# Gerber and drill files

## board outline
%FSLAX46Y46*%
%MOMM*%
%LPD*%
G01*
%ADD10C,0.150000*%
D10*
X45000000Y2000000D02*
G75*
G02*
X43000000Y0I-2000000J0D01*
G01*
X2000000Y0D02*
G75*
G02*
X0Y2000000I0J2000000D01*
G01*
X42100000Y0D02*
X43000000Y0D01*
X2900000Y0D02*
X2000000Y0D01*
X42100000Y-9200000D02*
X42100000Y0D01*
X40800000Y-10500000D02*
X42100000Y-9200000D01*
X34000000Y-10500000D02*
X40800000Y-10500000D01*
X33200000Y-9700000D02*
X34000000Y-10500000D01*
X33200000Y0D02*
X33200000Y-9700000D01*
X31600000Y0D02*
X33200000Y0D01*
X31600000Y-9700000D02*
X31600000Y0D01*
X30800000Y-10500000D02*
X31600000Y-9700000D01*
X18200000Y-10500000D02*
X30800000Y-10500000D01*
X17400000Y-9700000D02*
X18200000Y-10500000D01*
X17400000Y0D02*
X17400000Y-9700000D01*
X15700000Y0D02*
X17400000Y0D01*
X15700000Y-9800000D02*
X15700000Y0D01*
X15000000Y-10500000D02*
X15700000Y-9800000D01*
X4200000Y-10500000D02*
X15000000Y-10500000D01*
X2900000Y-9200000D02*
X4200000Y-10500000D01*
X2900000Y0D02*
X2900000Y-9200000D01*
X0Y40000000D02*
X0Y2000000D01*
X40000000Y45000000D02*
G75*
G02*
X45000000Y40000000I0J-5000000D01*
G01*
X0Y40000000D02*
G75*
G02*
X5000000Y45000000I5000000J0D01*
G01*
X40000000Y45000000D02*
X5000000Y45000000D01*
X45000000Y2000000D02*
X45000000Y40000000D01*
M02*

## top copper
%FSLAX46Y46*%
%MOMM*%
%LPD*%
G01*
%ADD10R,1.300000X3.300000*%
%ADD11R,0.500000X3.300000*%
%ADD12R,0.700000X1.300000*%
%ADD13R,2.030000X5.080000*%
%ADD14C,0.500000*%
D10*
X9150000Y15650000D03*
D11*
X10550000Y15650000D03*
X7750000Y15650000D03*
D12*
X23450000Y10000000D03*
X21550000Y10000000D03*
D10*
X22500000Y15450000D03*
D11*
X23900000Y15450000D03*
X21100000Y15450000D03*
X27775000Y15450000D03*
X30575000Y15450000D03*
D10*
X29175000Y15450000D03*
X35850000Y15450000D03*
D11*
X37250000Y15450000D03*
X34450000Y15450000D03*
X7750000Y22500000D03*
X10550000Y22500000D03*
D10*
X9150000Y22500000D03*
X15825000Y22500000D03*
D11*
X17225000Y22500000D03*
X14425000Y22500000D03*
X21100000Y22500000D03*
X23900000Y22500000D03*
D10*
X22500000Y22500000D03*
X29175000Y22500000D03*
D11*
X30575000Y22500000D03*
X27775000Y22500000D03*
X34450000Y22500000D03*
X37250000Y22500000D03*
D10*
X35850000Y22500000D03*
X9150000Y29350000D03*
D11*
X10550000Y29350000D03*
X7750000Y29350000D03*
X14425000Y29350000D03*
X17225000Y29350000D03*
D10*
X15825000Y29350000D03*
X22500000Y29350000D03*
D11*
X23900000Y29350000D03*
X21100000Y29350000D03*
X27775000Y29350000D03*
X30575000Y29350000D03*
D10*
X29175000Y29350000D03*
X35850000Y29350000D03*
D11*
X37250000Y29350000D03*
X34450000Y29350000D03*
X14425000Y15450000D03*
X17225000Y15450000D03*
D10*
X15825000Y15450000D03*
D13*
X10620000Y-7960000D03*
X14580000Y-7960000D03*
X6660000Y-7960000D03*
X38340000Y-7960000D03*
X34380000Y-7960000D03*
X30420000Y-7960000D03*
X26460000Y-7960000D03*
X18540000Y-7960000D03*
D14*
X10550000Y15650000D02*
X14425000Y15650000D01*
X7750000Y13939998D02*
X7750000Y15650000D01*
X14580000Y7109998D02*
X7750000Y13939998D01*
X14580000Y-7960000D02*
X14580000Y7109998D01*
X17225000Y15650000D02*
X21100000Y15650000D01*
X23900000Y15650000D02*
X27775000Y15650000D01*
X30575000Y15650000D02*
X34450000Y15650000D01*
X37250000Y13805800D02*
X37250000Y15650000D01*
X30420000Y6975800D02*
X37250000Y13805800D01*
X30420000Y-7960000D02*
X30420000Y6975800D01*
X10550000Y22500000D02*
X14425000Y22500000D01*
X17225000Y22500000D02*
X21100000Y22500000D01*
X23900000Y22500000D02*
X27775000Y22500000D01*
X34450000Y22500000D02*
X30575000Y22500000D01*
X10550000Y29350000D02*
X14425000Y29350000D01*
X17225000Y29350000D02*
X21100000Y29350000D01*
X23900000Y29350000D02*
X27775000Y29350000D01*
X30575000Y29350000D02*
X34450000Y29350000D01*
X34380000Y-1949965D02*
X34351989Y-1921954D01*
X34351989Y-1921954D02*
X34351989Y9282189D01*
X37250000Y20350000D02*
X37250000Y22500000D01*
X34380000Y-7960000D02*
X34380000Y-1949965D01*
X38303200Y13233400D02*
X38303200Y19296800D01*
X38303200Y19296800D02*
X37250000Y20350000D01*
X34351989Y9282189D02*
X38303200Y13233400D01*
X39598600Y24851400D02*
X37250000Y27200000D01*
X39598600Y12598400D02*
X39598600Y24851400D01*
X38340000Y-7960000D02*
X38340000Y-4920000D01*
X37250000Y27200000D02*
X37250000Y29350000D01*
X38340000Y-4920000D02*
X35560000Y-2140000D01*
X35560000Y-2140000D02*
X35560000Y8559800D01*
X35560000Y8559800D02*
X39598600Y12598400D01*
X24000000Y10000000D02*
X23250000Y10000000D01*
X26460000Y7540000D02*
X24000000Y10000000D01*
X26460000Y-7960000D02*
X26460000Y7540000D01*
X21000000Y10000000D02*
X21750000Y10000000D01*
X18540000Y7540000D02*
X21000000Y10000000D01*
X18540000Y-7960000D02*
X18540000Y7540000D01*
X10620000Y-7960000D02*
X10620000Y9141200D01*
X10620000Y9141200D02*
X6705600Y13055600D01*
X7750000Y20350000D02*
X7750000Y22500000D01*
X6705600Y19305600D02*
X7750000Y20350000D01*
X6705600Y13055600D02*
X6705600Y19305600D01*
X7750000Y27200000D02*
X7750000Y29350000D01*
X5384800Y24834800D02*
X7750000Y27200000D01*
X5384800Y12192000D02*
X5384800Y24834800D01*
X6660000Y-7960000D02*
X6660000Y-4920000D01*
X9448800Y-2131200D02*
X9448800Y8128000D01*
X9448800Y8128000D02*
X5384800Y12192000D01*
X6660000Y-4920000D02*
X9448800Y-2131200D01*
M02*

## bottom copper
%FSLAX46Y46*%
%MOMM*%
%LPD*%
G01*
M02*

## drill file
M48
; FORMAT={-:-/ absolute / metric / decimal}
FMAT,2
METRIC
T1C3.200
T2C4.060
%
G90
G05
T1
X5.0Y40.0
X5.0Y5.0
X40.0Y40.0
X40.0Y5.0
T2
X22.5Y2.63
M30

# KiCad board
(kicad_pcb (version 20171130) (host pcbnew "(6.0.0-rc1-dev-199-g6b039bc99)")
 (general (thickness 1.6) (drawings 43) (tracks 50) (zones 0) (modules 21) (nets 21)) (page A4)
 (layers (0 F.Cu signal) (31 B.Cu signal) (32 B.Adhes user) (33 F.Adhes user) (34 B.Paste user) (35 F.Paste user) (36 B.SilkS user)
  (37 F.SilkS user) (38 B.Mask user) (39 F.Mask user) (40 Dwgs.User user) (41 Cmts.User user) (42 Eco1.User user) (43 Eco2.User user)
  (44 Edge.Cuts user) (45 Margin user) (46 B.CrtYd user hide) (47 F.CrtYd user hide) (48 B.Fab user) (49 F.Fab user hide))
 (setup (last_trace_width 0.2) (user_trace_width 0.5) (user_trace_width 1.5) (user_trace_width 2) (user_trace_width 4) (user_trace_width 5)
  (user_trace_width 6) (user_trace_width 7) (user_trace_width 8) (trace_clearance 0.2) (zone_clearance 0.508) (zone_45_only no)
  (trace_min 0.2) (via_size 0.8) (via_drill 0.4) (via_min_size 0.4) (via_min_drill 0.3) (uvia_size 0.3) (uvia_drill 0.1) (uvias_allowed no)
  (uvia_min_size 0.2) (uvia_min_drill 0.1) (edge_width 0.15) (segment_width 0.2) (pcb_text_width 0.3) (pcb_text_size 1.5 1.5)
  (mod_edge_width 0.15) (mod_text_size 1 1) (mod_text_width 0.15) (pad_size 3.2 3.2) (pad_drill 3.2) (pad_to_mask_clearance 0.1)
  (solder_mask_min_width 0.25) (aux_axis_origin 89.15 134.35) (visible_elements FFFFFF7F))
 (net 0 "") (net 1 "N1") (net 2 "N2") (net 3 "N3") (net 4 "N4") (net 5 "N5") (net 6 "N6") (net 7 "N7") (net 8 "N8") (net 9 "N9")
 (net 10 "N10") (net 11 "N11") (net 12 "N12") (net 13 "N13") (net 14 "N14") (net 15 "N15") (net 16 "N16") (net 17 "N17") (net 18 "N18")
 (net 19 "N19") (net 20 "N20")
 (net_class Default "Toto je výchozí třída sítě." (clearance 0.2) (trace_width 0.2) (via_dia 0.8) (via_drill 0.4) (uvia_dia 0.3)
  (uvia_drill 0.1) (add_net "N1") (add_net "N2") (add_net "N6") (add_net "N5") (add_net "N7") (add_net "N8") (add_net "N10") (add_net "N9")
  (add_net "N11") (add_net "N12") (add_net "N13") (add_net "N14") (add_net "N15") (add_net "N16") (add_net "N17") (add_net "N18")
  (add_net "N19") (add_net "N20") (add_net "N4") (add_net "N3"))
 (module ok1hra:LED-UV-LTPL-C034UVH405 (layer F.Cu) (at 9.15 -15.65 180)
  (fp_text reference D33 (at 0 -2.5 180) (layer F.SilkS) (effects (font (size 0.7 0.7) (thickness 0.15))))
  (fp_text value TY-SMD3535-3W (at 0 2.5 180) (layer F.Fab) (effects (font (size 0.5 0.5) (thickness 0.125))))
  (pad 3 smd rect (at 0 0 180) (size 1.3 3.3) (layers F.Cu F.Paste F.Mask))
  (pad 1 smd rect (at -1.4 0 180) (size 0.5 3.3) (layers F.Cu F.Paste F.Mask) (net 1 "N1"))
  (pad 2 smd rect (at 1.4 0 180) (size 0.5 3.3) (layers F.Cu F.Paste F.Mask) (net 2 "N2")))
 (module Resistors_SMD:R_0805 (layer F.Cu) (at 22.5 -10 180)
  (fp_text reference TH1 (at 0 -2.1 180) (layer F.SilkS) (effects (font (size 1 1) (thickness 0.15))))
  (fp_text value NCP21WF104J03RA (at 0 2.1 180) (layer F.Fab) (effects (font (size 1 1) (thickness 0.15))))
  (pad 1 smd rect (at -0.95 0 180) (size 0.7 1.3) (layers F.Cu F.Paste F.Mask) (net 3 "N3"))
  (pad 2 smd rect (at 0.95 0 180) (size 0.7 1.3) (layers F.Cu F.Paste F.Mask) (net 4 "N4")))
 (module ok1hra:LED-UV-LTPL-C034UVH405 (layer F.Cu) (at 22.5 -15.45 180)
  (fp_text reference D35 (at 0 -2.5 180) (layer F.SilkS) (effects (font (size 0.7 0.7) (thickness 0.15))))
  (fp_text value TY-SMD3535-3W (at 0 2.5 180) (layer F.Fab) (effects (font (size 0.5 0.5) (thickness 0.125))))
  (pad 3 smd rect (at 0 0 180) (size 1.3 3.3) (layers F.Cu F.Paste F.Mask))
  (pad 1 smd rect (at -1.4 0 180) (size 0.5 3.3) (layers F.Cu F.Paste F.Mask) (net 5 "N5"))
  (pad 2 smd rect (at 1.4 0 180) (size 0.5 3.3) (layers F.Cu F.Paste F.Mask) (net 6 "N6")))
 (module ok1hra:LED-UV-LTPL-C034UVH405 (layer F.Cu) (at 29.175 -15.45 180)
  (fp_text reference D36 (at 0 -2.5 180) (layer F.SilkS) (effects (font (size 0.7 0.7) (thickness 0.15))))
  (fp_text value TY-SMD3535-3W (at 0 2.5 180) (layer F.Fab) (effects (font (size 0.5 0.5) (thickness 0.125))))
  (pad 2 smd rect (at 1.4 0 180) (size 0.5 3.3) (layers F.Cu F.Paste F.Mask) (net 5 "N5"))
  (pad 1 smd rect (at -1.4 0 180) (size 0.5 3.3) (layers F.Cu F.Paste F.Mask) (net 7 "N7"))
  (pad 3 smd rect (at 0 0 180) (size 1.3 3.3) (layers F.Cu F.Paste F.Mask)))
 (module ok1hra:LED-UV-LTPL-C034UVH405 (layer F.Cu) (at 35.85 -15.45 180)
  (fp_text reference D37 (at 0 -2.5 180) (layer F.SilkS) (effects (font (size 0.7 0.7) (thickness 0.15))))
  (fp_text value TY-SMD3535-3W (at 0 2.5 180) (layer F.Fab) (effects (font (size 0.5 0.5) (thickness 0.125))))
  (pad 3 smd rect (at 0 0 180) (size 1.3 3.3) (layers F.Cu F.Paste F.Mask))
  (pad 1 smd rect (at -1.4 0 180) (size 0.5 3.3) (layers F.Cu F.Paste F.Mask) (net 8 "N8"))
  (pad 2 smd rect (at 1.4 0 180) (size 0.5 3.3) (layers F.Cu F.Paste F.Mask) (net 7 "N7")))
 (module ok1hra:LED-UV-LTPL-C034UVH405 (layer F.Cu) (at 9.15 -22.5 180)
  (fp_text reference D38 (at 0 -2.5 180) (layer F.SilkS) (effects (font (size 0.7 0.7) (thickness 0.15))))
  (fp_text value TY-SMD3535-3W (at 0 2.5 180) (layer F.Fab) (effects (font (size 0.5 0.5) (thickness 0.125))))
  (pad 2 smd rect (at 1.4 0 180) (size 0.5 3.3) (layers F.Cu F.Paste F.Mask) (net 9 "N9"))
  (pad 1 smd rect (at -1.4 0 180) (size 0.5 3.3) (layers F.Cu F.Paste F.Mask) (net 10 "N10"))
  (pad 3 smd rect (at 0 0 180) (size 1.3 3.3) (layers F.Cu F.Paste F.Mask)))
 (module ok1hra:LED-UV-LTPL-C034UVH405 (layer F.Cu) (at 15.825 -22.5 180)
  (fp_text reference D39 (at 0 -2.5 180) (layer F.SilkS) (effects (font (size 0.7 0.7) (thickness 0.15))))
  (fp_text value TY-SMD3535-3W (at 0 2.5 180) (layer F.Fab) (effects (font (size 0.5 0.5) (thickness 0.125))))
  (pad 3 smd rect (at 0 0 180) (size 1.3 3.3) (layers F.Cu F.Paste F.Mask))
  (pad 1 smd rect (at -1.4 0 180) (size 0.5 3.3) (layers F.Cu F.Paste F.Mask) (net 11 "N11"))
  (pad 2 smd rect (at 1.4 0 180) (size 0.5 3.3) (layers F.Cu F.Paste F.Mask) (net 10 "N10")))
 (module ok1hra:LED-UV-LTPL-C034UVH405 (layer F.Cu) (at 22.5 -22.5 180)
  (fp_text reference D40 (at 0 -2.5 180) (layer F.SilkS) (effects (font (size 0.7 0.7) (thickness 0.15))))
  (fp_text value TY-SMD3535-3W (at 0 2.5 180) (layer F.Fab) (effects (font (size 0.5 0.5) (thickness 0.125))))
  (pad 2 smd rect (at 1.4 0 180) (size 0.5 3.3) (layers F.Cu F.Paste F.Mask) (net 11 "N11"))
  (pad 1 smd rect (at -1.4 0 180) (size 0.5 3.3) (layers F.Cu F.Paste F.Mask) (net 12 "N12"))
  (pad 3 smd rect (at 0 0 180) (size 1.3 3.3) (layers F.Cu F.Paste F.Mask)))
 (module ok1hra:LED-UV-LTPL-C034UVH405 (layer F.Cu) (at 29.175 -22.5 180)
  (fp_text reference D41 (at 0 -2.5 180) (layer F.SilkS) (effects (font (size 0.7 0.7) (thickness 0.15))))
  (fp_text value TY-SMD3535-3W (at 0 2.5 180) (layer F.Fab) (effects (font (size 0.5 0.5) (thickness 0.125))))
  (pad 3 smd rect (at 0 0 180) (size 1.3 3.3) (layers F.Cu F.Paste F.Mask))
  (pad 1 smd rect (at -1.4 0 180) (size 0.5 3.3) (layers F.Cu F.Paste F.Mask) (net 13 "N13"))
  (pad 2 smd rect (at 1.4 0 180) (size 0.5 3.3) (layers F.Cu F.Paste F.Mask) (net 12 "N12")))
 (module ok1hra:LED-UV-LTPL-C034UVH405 (layer F.Cu) (at 35.85 -22.5 180)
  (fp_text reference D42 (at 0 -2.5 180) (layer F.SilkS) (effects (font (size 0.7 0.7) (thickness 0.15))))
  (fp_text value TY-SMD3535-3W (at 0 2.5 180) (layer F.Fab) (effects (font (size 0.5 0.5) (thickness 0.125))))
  (pad 2 smd rect (at 1.4 0 180) (size 0.5 3.3) (layers F.Cu F.Paste F.Mask) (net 13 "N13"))
  (pad 1 smd rect (at -1.4 0 180) (size 0.5 3.3) (layers F.Cu F.Paste F.Mask) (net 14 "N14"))
  (pad 3 smd rect (at 0 0 180) (size 1.3 3.3) (layers F.Cu F.Paste F.Mask)))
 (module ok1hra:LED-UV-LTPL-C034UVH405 (layer F.Cu) (at 9.15 -29.35 180)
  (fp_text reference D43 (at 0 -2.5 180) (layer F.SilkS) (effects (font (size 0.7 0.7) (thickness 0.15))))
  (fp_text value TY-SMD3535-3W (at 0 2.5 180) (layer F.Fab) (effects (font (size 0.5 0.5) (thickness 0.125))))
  (pad 3 smd rect (at 0 0 180) (size 1.3 3.3) (layers F.Cu F.Paste F.Mask))
  (pad 1 smd rect (at -1.4 0 180) (size 0.5 3.3) (layers F.Cu F.Paste F.Mask) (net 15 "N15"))
  (pad 2 smd rect (at 1.4 0 180) (size 0.5 3.3) (layers F.Cu F.Paste F.Mask) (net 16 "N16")))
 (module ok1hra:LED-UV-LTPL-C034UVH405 (layer F.Cu) (at 15.825 -29.35 180)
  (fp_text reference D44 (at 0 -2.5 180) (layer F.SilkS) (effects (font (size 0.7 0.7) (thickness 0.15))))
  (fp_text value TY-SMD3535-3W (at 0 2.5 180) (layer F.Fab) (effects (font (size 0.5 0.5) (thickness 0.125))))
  (pad 2 smd rect (at 1.4 0 180) (size 0.5 3.3) (layers F.Cu F.Paste F.Mask) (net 15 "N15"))
  (pad 1 smd rect (at -1.4 0 180) (size 0.5 3.3) (layers F.Cu F.Paste F.Mask) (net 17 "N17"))
  (pad 3 smd rect (at 0 0 180) (size 1.3 3.3) (layers F.Cu F.Paste F.Mask)))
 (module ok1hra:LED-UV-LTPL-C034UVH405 (layer F.Cu) (at 22.5 -29.35 180)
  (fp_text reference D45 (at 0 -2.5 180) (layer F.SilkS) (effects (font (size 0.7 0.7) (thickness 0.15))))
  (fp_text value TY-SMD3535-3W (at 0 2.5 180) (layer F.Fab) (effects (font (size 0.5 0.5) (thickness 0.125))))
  (pad 3 smd rect (at 0 0 180) (size 1.3 3.3) (layers F.Cu F.Paste F.Mask))
  (pad 1 smd rect (at -1.4 0 180) (size 0.5 3.3) (layers F.Cu F.Paste F.Mask) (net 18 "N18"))
  (pad 2 smd rect (at 1.4 0 180) (size 0.5 3.3) (layers F.Cu F.Paste F.Mask) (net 17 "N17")))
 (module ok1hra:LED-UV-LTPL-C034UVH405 (layer F.Cu) (at 29.175 -29.35 180)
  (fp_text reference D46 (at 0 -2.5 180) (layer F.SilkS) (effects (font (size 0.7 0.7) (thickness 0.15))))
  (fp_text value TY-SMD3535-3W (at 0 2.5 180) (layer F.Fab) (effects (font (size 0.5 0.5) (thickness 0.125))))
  (pad 2 smd rect (at 1.4 0 180) (size 0.5 3.3) (layers F.Cu F.Paste F.Mask) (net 18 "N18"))
  (pad 1 smd rect (at -1.4 0 180) (size 0.5 3.3) (layers F.Cu F.Paste F.Mask) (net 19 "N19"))
  (pad 3 smd rect (at 0 0 180) (size 1.3 3.3) (layers F.Cu F.Paste F.Mask)))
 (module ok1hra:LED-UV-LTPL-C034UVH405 (layer F.Cu) (at 35.85 -29.35 180)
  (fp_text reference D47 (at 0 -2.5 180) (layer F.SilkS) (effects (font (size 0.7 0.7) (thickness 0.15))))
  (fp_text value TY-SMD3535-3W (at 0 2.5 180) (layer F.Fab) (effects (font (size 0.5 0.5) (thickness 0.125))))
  (pad 3 smd rect (at 0 0 180) (size 1.3 3.3) (layers F.Cu F.Paste F.Mask))
  (pad 1 smd rect (at -1.4 0 180) (size 0.5 3.3) (layers F.Cu F.Paste F.Mask) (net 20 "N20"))
  (pad 2 smd rect (at 1.4 0 180) (size 0.5 3.3) (layers F.Cu F.Paste F.Mask) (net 19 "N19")))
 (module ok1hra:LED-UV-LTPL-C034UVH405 (layer F.Cu) (at 15.825 -15.45 180)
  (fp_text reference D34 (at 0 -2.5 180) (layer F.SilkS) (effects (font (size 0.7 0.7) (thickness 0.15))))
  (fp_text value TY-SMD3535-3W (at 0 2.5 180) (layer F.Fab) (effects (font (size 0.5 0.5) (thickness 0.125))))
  (pad 2 smd rect (at 1.4 0 180) (size 0.5 3.3) (layers F.Cu F.Paste F.Mask) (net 1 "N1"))
  (pad 1 smd rect (at -1.4 0 180) (size 0.5 3.3) (layers F.Cu F.Paste F.Mask) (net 6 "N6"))
  (pad 3 smd rect (at 0 0 180) (size 1.3 3.3) (layers F.Cu F.Paste F.Mask)))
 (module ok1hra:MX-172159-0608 (layer F.Cu) (at 22.5 10.5 180)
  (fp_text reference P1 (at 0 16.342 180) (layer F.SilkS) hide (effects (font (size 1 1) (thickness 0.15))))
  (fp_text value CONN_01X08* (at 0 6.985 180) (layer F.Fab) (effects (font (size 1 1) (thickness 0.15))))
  (pad 2 smd rect (at 11.88 2.54 180) (size 2.03 5.08) (layers F.Cu F.Mask) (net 9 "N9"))
  (pad 3 smd rect (at 7.92 2.54 180) (size 2.03 5.08) (layers F.Cu F.Mask) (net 2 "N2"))
  (pad 1 smd rect (at 15.84 2.54 180) (size 2.03 5.08) (layers F.Cu F.Mask) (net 16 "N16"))
  (pad 8 smd rect (at -15.84 2.54 180) (size 2.03 5.08) (layers F.Cu F.Mask) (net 20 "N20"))
  (pad 7 smd rect (at -11.88 2.54 180) (size 2.03 5.08) (layers F.Cu F.Mask) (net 14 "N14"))
  (pad 6 smd rect (at -7.92 2.54 180) (size 2.03 5.08) (layers F.Cu F.Mask) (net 8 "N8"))
  (pad 5 smd rect (at -3.96 2.54 180) (size 2.03 5.08) (layers F.Cu F.Mask) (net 3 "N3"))
  (pad 4 smd rect (at 3.96 2.54 180) (size 2.03 5.08) (layers F.Cu F.Mask) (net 4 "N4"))
  (pad "" np_thru_hole circle (at 0 13.13 180) (size 4.06 4.06) (drill 4.06) (layers *.Cu *.Mask)))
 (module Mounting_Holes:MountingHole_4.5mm (layer F.Cu) (at 40 -40)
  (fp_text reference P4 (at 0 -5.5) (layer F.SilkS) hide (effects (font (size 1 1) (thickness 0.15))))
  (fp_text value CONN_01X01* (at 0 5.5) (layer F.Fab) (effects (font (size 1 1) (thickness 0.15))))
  (pad "" np_thru_hole circle (at 0 0) (size 3.2 3.2) (drill 3.2) (layers *.Cu *.Mask)))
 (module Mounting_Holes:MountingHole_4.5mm (layer F.Cu) (at 40 -5)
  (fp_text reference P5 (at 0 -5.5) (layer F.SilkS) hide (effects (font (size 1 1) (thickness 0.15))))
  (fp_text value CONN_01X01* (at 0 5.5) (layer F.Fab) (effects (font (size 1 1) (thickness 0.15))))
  (pad "" np_thru_hole circle (at 0 0) (size 3.2 3.2) (drill 3.2) (layers *.Cu *.Mask)))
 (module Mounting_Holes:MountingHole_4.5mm (layer F.Cu) (at 5 -5)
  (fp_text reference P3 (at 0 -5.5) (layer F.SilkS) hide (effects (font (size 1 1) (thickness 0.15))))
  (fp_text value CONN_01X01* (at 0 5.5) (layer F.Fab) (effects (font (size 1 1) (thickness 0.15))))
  (pad "" np_thru_hole circle (at 0 0) (size 3.2 3.2) (drill 3.2) (layers *.Cu *.Mask)))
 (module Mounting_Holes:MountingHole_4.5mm (layer F.Cu) (at 5 -40)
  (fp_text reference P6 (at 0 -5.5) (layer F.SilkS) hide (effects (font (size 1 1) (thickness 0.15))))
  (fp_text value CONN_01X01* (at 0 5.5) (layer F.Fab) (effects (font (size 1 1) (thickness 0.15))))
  (pad "" np_thru_hole circle (at 0 0) (size 3.2 3.2) (drill 3.2) (layers *.Cu *.Mask)))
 (gr_arc (start 43 -2) (end 43 0) (angle -90) (layer Edge.Cuts) (width 0.15))
 (gr_arc (start 2 -2) (end 0 -2) (angle -90) (layer Edge.Cuts) (width 0.15))
 (gr_line (start 42.1 0) (end 43 0) (layer Edge.Cuts) (width 0.15))
 (gr_line (start 2.9 0) (end 2 0) (layer Edge.Cuts) (width 0.15))
 (gr_line (start 42.1 9.2) (end 42.1 0) (layer Edge.Cuts) (width 0.15))
 (gr_line (start 40.8 10.5) (end 42.1 9.2) (layer Edge.Cuts) (width 0.15))
 (gr_line (start 34 10.5) (end 40.8 10.5) (layer Edge.Cuts) (width 0.15))
 (gr_line (start 33.2 9.7) (end 34 10.5) (layer Edge.Cuts) (width 0.15))
 (gr_line (start 33.2 0) (end 33.2 9.7) (layer Edge.Cuts) (width 0.15))
 (gr_line (start 31.6 0) (end 33.2 0) (layer Edge.Cuts) (width 0.15))
 (gr_line (start 31.6 9.7) (end 31.6 0) (layer Edge.Cuts) (width 0.15))
 (gr_line (start 30.8 10.5) (end 31.6 9.7) (layer Edge.Cuts) (width 0.15))
 (gr_line (start 18.2 10.5) (end 30.8 10.5) (layer Edge.Cuts) (width 0.15))
 (gr_line (start 17.4 9.7) (end 18.2 10.5) (layer Edge.Cuts) (width 0.15))
 (gr_line (start 17.4 0) (end 17.4 9.7) (layer Edge.Cuts) (width 0.15))
 (gr_line (start 15.7 0) (end 17.4 0) (layer Edge.Cuts) (width 0.15))
 (gr_line (start 15.7 9.8) (end 15.7 0) (layer Edge.Cuts) (width 0.15))
 (gr_line (start 15 10.5) (end 15.7 9.8) (layer Edge.Cuts) (width 0.15))
 (gr_line (start 4.2 10.5) (end 15 10.5) (layer Edge.Cuts) (width 0.15))
 (gr_line (start 2.9 9.2) (end 4.2 10.5) (layer Edge.Cuts) (width 0.15))
 (gr_line (start 2.9 0) (end 2.9 9.2) (layer Edge.Cuts) (width 0.15))
 (gr_line (start 0 -40) (end 0 -2) (layer Edge.Cuts) (width 0.15))
 (gr_arc (start 40 -40) (end 45 -40) (angle -90) (layer Edge.Cuts) (width 0.15))
 (gr_arc (start 5 -40) (end 5 -45) (angle -90) (layer Edge.Cuts) (width 0.15))
 (gr_line (start 40 -45) (end 5 -45) (layer Edge.Cuts) (width 0.15))
 (gr_line (start 45 -2) (end 45 -40) (layer Edge.Cuts) (width 0.15))
 (segment (start 10.55 -15.65) (end 14.425 -15.65) (width 0.5) (layer F.Cu) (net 1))
 (segment (start 7.75 -13.939998) (end 7.75 -15.65) (width 0.5) (layer F.Cu) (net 2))
 (segment (start 14.58 -7.109998) (end 7.75 -13.939998) (width 0.5) (layer F.Cu) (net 2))
 (segment (start 14.58 7.96) (end 14.58 -7.109998) (width 0.5) (layer F.Cu) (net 2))
 (segment (start 17.225 -15.65) (end 21.1 -15.65) (width 0.5) (layer F.Cu) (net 6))
 (segment (start 23.9 -15.65) (end 27.775 -15.65) (width 0.5) (layer F.Cu) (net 5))
 (segment (start 30.575 -15.65) (end 34.45 -15.65) (width 0.5) (layer F.Cu) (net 7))
 (segment (start 37.25 -13.8058) (end 37.25 -15.65) (width 0.5) (layer F.Cu) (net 8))
 (segment (start 30.42 -6.9758) (end 37.25 -13.8058) (width 0.5) (layer F.Cu) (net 8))
 (segment (start 30.42 7.96) (end 30.42 -6.9758) (width 0.5) (layer F.Cu) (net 8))
 (segment (start 10.55 -22.5) (end 14.425 -22.5) (width 0.5) (layer F.Cu) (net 10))
 (segment (start 17.225 -22.5) (end 21.1 -22.5) (width 0.5) (layer F.Cu) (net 11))
 (segment (start 23.9 -22.5) (end 27.775 -22.5) (width 0.5) (layer F.Cu) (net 12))
 (segment (start 34.45 -22.5) (end 30.575 -22.5) (width 0.5) (layer F.Cu) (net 13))
 (segment (start 10.55 -29.35) (end 14.425 -29.35) (width 0.5) (layer F.Cu) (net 15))
 (segment (start 17.225 -29.35) (end 21.1 -29.35) (width 0.5) (layer F.Cu) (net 17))
 (segment (start 23.9 -29.35) (end 27.775 -29.35) (width 0.5) (layer F.Cu) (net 18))
 (segment (start 30.575 -29.35) (end 34.45 -29.35) (width 0.5) (layer F.Cu) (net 19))
 (segment (start 34.38 1.949965) (end 34.351989 1.921954) (width 0.5) (layer F.Cu) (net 14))
 (segment (start 34.351989 1.921954) (end 34.351989 -9.282189) (width 0.5) (layer F.Cu) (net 14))
 (segment (start 37.25 -20.35) (end 37.25 -22.5) (width 0.5) (layer F.Cu) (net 14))
 (segment (start 34.38 7.96) (end 34.38 1.949965) (width 0.5) (layer F.Cu) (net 14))
 (segment (start 38.3032 -13.2334) (end 38.3032 -19.2968) (width 0.5) (layer F.Cu) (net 14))
 (segment (start 38.3032 -19.2968) (end 37.25 -20.35) (width 0.5) (layer F.Cu) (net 14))
 (segment (start 34.351989 -9.282189) (end 38.3032 -13.2334) (width 0.5) (layer F.Cu) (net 14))
 (segment (start 39.5986 -24.8514) (end 37.25 -27.2) (width 0.5) (layer F.Cu) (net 20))
 (segment (start 39.5986 -12.5984) (end 39.5986 -24.8514) (width 0.5) (layer F.Cu) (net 20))
 (segment (start 38.34 7.96) (end 38.34 4.92) (width 0.5) (layer F.Cu) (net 20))
 (segment (start 37.25 -27.2) (end 37.25 -29.35) (width 0.5) (layer F.Cu) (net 20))
 (segment (start 38.34 4.92) (end 35.56 2.14) (width 0.5) (layer F.Cu) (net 20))
 (segment (start 35.56 2.14) (end 35.56 -8.5598) (width 0.5) (layer F.Cu) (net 20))
 (segment (start 35.56 -8.5598) (end 39.5986 -12.5984) (width 0.5) (layer F.Cu) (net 20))
 (segment (start 24 -10) (end 23.25 -10) (width 0.5) (layer F.Cu) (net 3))
 (segment (start 26.46 -7.54) (end 24 -10) (width 0.5) (layer F.Cu) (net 3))
 (segment (start 26.46 7.96) (end 26.46 -7.54) (width 0.5) (layer F.Cu) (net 3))
 (segment (start 21 -10) (end 21.75 -10) (width 0.5) (layer F.Cu) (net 4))
 (segment (start 18.54 -7.54) (end 21 -10) (width 0.5) (layer F.Cu) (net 4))
 (segment (start 18.54 7.96) (end 18.54 -7.54) (width 0.5) (layer F.Cu) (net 4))
 (segment (start 10.62 7.96) (end 10.62 -9.1412) (width 0.5) (layer F.Cu) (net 9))
 (segment (start 10.62 -9.1412) (end 6.7056 -13.0556) (width 0.5) (layer F.Cu) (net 9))
 (segment (start 7.75 -20.35) (end 7.75 -22.5) (width 0.5) (layer F.Cu) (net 9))
 (segment (start 6.7056 -19.3056) (end 7.75 -20.35) (width 0.5) (layer F.Cu) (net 9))
 (segment (start 6.7056 -13.0556) (end 6.7056 -19.3056) (width 0.5) (layer F.Cu) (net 9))
 (segment (start 7.75 -27.2) (end 7.75 -29.35) (width 0.5) (layer F.Cu) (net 16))
 (segment (start 5.3848 -24.8348) (end 7.75 -27.2) (width 0.5) (layer F.Cu) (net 16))
 (segment (start 5.3848 -12.192) (end 5.3848 -24.8348) (width 0.5) (layer F.Cu) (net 16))
 (segment (start 6.66 7.96) (end 6.66 4.92) (width 0.5) (layer F.Cu) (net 16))
 (segment (start 9.4488 2.1312) (end 9.4488 -8.128) (width 0.5) (layer F.Cu) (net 16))
 (segment (start 9.4488 -8.128) (end 5.3848 -12.192) (width 0.5) (layer F.Cu) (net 16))
 (segment (start 6.66 4.92) (end 9.4488 2.1312) (width 0.5) (layer F.Cu) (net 16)))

